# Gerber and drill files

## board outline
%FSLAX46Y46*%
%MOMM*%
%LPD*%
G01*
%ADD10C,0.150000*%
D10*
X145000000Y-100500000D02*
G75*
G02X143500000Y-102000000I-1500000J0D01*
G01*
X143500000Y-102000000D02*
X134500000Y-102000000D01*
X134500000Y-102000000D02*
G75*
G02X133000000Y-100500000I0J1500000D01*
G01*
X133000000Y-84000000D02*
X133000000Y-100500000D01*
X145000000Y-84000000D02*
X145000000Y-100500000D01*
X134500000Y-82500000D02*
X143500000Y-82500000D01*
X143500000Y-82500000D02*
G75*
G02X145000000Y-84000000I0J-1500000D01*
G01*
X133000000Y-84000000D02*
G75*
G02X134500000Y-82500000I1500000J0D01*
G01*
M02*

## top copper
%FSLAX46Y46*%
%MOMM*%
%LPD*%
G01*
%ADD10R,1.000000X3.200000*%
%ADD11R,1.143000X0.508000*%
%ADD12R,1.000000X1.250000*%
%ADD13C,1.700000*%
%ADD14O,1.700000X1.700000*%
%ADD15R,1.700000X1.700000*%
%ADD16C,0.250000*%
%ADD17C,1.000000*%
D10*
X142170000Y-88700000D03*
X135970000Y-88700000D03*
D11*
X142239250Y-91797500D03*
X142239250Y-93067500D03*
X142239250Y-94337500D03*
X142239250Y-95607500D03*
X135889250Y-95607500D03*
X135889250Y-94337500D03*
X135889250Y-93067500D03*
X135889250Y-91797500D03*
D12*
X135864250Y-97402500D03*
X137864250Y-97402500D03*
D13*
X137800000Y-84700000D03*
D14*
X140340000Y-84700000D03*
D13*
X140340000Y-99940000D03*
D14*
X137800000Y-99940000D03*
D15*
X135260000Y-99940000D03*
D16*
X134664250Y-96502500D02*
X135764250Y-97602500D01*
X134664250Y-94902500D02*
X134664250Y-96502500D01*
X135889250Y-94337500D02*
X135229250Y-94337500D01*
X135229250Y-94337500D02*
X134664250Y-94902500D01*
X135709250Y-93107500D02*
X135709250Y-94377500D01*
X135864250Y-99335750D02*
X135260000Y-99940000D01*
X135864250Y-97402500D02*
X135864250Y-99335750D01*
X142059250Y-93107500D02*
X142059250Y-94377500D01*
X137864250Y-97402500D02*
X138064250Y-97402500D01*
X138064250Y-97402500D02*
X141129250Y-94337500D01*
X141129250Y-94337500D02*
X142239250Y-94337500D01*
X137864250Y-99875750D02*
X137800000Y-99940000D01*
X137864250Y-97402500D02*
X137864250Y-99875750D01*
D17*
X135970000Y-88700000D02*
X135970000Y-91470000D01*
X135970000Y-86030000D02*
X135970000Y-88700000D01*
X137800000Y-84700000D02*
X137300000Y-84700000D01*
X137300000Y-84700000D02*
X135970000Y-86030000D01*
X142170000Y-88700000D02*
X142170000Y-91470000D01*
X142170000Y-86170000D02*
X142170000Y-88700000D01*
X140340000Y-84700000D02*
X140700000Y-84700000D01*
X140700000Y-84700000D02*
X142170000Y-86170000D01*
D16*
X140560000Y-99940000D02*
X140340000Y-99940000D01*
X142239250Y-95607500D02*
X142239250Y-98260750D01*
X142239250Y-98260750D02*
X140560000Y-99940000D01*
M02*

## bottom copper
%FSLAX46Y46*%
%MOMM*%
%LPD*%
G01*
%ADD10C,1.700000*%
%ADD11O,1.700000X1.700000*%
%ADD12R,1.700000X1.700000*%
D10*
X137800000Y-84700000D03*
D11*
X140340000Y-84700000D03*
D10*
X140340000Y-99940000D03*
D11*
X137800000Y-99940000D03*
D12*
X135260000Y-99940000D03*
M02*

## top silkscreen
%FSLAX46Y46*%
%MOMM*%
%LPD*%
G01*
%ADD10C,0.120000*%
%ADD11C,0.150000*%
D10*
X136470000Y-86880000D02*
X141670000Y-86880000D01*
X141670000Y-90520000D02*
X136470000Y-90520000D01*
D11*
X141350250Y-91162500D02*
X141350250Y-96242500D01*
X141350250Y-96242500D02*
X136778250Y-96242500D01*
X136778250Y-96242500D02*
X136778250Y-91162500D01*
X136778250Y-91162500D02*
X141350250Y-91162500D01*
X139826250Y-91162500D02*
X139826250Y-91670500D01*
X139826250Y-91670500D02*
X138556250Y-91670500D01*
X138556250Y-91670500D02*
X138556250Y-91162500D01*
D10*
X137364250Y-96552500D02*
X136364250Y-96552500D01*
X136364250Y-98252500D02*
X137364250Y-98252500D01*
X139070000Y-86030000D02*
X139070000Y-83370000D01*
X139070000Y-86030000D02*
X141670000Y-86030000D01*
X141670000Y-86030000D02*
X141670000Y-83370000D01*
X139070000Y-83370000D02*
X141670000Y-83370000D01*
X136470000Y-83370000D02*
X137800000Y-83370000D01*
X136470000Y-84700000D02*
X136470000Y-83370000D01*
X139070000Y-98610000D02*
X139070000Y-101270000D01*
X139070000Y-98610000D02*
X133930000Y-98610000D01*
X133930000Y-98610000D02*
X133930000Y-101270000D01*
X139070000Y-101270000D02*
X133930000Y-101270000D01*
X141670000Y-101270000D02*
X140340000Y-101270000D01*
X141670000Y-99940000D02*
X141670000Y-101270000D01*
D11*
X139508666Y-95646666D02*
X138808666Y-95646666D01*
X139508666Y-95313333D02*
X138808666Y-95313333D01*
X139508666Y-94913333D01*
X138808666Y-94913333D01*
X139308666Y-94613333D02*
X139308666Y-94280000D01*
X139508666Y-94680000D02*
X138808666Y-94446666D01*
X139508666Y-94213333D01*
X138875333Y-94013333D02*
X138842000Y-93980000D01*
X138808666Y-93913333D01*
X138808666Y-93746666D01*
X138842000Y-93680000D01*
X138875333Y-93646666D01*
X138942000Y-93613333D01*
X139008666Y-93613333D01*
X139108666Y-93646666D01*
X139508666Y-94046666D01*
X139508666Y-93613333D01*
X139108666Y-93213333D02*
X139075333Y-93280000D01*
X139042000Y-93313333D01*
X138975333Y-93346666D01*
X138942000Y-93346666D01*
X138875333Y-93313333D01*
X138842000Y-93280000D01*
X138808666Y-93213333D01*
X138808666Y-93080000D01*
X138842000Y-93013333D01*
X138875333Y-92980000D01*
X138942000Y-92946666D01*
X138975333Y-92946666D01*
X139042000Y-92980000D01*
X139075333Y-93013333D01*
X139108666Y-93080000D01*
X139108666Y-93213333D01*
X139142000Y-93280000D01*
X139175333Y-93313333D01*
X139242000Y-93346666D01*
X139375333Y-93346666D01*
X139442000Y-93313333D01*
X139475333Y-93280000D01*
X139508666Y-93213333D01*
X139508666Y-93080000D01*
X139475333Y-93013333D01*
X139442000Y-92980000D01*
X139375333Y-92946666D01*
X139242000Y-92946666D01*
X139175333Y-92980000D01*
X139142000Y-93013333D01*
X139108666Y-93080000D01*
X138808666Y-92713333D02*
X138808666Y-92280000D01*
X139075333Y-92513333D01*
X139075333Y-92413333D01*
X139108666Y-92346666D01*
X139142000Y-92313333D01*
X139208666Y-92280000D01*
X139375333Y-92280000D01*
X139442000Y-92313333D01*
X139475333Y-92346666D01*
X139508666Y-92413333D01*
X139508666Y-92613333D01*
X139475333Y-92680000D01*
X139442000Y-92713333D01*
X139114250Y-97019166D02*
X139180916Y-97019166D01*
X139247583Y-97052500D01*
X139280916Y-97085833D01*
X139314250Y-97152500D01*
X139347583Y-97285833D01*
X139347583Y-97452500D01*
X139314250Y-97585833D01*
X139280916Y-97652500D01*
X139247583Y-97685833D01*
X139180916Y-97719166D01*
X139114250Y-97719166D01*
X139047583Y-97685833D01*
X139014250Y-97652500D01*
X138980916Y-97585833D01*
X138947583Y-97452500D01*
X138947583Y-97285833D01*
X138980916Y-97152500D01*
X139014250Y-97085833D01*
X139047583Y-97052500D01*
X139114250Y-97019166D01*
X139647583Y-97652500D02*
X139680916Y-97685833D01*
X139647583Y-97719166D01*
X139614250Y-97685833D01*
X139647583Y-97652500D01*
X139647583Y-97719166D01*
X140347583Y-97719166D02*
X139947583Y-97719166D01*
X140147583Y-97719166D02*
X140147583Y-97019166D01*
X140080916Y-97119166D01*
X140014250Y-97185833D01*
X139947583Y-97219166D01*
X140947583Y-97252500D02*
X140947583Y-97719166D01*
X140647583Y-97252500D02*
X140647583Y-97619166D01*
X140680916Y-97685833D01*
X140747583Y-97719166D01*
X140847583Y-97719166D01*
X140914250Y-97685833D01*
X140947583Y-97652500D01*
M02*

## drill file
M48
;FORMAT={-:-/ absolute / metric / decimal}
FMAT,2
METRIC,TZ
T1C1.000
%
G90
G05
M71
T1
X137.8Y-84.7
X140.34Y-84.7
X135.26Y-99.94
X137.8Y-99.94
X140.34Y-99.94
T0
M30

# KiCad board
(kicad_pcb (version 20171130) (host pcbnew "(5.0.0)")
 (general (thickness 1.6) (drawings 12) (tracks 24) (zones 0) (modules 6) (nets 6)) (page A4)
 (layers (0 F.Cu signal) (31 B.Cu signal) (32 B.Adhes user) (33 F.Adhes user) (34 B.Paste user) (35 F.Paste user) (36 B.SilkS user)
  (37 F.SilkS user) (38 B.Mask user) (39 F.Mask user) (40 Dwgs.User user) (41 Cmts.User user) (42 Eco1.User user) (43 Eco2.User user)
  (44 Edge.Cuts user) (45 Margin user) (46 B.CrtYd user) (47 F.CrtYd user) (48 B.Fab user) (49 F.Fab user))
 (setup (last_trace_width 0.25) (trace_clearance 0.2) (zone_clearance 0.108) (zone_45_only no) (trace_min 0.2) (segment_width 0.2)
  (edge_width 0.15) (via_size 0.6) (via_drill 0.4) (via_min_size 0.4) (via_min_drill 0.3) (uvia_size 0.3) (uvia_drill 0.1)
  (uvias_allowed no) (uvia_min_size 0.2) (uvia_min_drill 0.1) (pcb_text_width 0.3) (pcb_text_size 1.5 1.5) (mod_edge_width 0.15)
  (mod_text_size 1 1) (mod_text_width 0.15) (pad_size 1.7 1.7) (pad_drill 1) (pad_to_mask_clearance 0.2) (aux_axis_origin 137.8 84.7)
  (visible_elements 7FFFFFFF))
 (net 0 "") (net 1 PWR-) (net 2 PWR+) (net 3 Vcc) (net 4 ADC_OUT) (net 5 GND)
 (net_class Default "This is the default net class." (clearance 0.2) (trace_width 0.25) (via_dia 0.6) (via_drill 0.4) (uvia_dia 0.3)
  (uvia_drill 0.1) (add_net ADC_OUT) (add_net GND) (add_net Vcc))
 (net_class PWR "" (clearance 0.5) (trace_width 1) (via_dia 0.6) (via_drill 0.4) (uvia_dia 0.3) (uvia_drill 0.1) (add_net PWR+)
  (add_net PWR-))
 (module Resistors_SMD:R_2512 (layer F.Cu) (at 139.07 88.7 180)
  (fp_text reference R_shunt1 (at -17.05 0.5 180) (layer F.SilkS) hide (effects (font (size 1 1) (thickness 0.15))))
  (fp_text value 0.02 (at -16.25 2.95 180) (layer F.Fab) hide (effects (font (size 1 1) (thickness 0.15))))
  (fp_line (start 2.6 1.82) (end -2.6 1.82) (layer F.SilkS) (width 0.12))
  (fp_line (start -2.6 -1.82) (end 2.6 -1.82) (layer F.SilkS) (width 0.12))
  (pad 1 smd rect (at -3.1 0 180) (size 1 3.2) (layers F.Cu F.Paste F.Mask) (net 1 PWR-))
  (pad 2 smd rect (at 3.1 0 180) (size 1 3.2) (layers F.Cu F.Paste F.Mask) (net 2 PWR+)))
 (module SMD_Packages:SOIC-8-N (layer F.Cu) (at 139.06425 93.7025 270)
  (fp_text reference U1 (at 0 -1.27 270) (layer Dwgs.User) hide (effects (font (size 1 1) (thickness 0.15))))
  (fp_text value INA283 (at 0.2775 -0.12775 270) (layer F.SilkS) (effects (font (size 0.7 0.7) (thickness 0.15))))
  (fp_line (start -2.54 -2.286) (end 2.54 -2.286) (layer F.SilkS) (width 0.15))
  (fp_line (start 2.54 -2.286) (end 2.54 2.286) (layer F.SilkS) (width 0.15))
  (fp_line (start 2.54 2.286) (end -2.54 2.286) (layer F.SilkS) (width 0.15))
  (fp_line (start -2.54 2.286) (end -2.54 -2.286) (layer F.SilkS) (width 0.15))
  (fp_line (start -2.54 -0.762) (end -2.032 -0.762) (layer F.SilkS) (width 0.15))
  (fp_line (start -2.032 -0.762) (end -2.032 0.508) (layer F.SilkS) (width 0.15))
  (fp_line (start -2.032 0.508) (end -2.54 0.508) (layer F.SilkS) (width 0.15))
  (pad 8 smd rect (at -1.905 -3.175 270) (size 0.508 1.143) (layers F.Cu F.Paste F.Mask) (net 1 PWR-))
  (pad 7 smd rect (at -0.635 -3.175 270) (size 0.508 1.143) (layers F.Cu F.Paste F.Mask) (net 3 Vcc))
  (pad 6 smd rect (at 0.635 -3.175 270) (size 0.508 1.143) (layers F.Cu F.Paste F.Mask) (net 3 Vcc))
  (pad 5 smd rect (at 1.905 -3.175 270) (size 0.508 1.143) (layers F.Cu F.Paste F.Mask) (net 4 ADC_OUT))
  (pad 4 smd rect (at 1.905 3.175 270) (size 0.508 1.143) (layers F.Cu F.Paste F.Mask))
  (pad 3 smd rect (at 0.635 3.175 270) (size 0.508 1.143) (layers F.Cu F.Paste F.Mask) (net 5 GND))
  (pad 2 smd rect (at -0.635 3.175 270) (size 0.508 1.143) (layers F.Cu F.Paste F.Mask) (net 5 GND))
  (pad 1 smd rect (at -1.905 3.175 270) (size 0.508 1.143) (layers F.Cu F.Paste F.Mask) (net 2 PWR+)))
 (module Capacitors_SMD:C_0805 (layer F.Cu) (at 136.86425 97.4025)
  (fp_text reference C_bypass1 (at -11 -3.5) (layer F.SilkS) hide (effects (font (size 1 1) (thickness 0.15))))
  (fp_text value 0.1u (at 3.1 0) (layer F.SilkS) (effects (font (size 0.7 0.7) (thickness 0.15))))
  (fp_line (start 0.5 -0.85) (end -0.5 -0.85) (layer F.SilkS) (width 0.12))
  (fp_line (start -0.5 0.85) (end 0.5 0.85) (layer F.SilkS) (width 0.12))
  (pad 1 smd rect (at -1 0) (size 1 1.25) (layers F.Cu F.Paste F.Mask) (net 5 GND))
  (pad 2 smd rect (at 1 0) (size 1 1.25) (layers F.Cu F.Paste F.Mask) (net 3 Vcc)))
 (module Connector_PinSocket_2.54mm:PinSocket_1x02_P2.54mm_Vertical (layer F.Cu) (at 137.8 84.7 90)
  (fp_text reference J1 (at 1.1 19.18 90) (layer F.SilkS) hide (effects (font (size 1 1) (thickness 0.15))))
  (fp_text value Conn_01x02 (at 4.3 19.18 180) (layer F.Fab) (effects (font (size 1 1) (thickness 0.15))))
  (fp_line (start -1.33 1.27) (end 1.33 1.27) (layer F.SilkS) (width 0.12))
  (fp_line (start -1.33 1.27) (end -1.33 3.87) (layer F.SilkS) (width 0.12))
  (fp_line (start -1.33 3.87) (end 1.33 3.87) (layer F.SilkS) (width 0.12))
  (fp_line (start 1.33 1.27) (end 1.33 3.87) (layer F.SilkS) (width 0.12))
  (fp_line (start 1.33 -1.33) (end 1.33 0) (layer F.SilkS) (width 0.12))
  (fp_line (start 0 -1.33) (end 1.33 -1.33) (layer F.SilkS) (width 0.12))
  (pad 1 thru_hole circle (at 0 0 90) (size 1.7 1.7) (drill 1) (layers *.Cu *.Mask) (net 2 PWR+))
  (pad 2 thru_hole oval (at 0 2.54 90) (size 1.7 1.7) (drill 1) (layers *.Cu *.Mask) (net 1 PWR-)))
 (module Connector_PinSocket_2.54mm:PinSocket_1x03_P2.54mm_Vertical (layer F.Cu) (at 140.34 99.94 270)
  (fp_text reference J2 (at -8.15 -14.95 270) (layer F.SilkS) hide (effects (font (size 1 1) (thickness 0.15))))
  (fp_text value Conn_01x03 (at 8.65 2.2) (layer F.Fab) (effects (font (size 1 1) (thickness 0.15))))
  (fp_line (start -1.33 1.27) (end 1.33 1.27) (layer F.SilkS) (width 0.12))
  (fp_line (start -1.33 1.27) (end -1.33 6.41) (layer F.SilkS) (width 0.12))
  (fp_line (start -1.33 6.41) (end 1.33 6.41) (layer F.SilkS) (width 0.12))
  (fp_line (start 1.33 1.27) (end 1.33 6.41) (layer F.SilkS) (width 0.12))
  (fp_line (start 1.33 -1.33) (end 1.33 0) (layer F.SilkS) (width 0.12))
  (fp_line (start 0 -1.33) (end 1.33 -1.33) (layer F.SilkS) (width 0.12))
  (pad 1 thru_hole circle (at 0 0 270) (size 1.7 1.7) (drill 1) (layers *.Cu *.Mask) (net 4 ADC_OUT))
  (pad 2 thru_hole oval (at 0 2.54 270) (size 1.7 1.7) (drill 1) (layers *.Cu *.Mask) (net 3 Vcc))
  (pad 3 thru_hole rect (at 0 5.08 270) (size 1.7 1.7) (drill 1) (layers *.Cu *.Mask) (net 5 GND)))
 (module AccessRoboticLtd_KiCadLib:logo (layer B.Cu) (at 139 90.5 180)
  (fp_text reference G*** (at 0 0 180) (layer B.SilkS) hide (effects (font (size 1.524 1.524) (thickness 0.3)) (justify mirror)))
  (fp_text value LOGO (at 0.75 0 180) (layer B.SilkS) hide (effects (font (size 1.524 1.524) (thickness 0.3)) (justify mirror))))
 (gr_arc (start 143.5 100.5) (end 143.5 102) (angle -90) (layer Edge.Cuts) (width 0.15))
 (gr_line (start 143.5 102) (end 134.5 102) (layer Edge.Cuts) (width 0.15))
 (gr_arc (start 134.5 100.5) (end 133 100.5) (angle -90) (layer Edge.Cuts) (width 0.15))
 (gr_line (start 133 84) (end 133 100.5) (layer Edge.Cuts) (width 0.15))
 (gr_line (start 145 84) (end 145 100.5) (layer Edge.Cuts) (width 0.15))
 (gr_line (start 134.5 82.5) (end 143.5 82.5) (layer Edge.Cuts) (width 0.15))
 (gr_arc (start 143.5 84) (end 145 84) (angle -90) (layer Edge.Cuts) (width 0.15))
 (gr_arc (start 134.5 84) (end 134.5 82.5) (angle -90) (layer Edge.Cuts) (width 0.15))
 (segment (start 134.66425 96.5025) (end 135.76425 97.6025) (width 0.25) (layer F.Cu) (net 5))
 (segment (start 134.66425 94.9025) (end 134.66425 96.5025) (width 0.25) (layer F.Cu) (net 5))
 (segment (start 135.88925 94.3375) (end 135.22925 94.3375) (width 0.25) (layer F.Cu) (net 5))
 (segment (start 135.22925 94.3375) (end 134.66425 94.9025) (width 0.25) (layer F.Cu) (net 5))
 (segment (start 135.70925 93.1075) (end 135.70925 94.3775) (width 0.25) (layer F.Cu) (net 5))
 (segment (start 135.86425 99.33575) (end 135.26 99.94) (width 0.25) (layer F.Cu) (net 5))
 (segment (start 135.86425 97.4025) (end 135.86425 99.33575) (width 0.25) (layer F.Cu) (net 5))
 (segment (start 142.05925 93.1075) (end 142.05925 94.3775) (width 0.25) (layer F.Cu) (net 3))
 (segment (start 137.86425 97.4025) (end 138.06425 97.4025) (width 0.25) (layer F.Cu) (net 3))
 (segment (start 138.06425 97.4025) (end 141.12925 94.3375) (width 0.25) (layer F.Cu) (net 3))
 (segment (start 141.12925 94.3375) (end 142.23925 94.3375) (width 0.25) (layer F.Cu) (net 3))
 (segment (start 137.86425 99.87575) (end 137.8 99.94) (width 0.25) (layer F.Cu) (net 3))
 (segment (start 137.86425 97.4025) (end 137.86425 99.87575) (width 0.25) (layer F.Cu) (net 3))
 (segment (start 135.97 88.7) (end 135.97 91.47) (width 1) (layer F.Cu) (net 2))
 (segment (start 135.97 86.03) (end 135.97 88.7) (width 1) (layer F.Cu) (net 2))
 (segment (start 137.8 84.7) (end 137.3 84.7) (width 1) (layer F.Cu) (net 2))
 (segment (start 137.3 84.7) (end 135.97 86.03) (width 1) (layer F.Cu) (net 2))
 (segment (start 142.17 88.7) (end 142.17 91.47) (width 1) (layer F.Cu) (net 1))
 (segment (start 142.17 86.17) (end 142.17 88.7) (width 1) (layer F.Cu) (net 1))
 (segment (start 140.34 84.7) (end 140.7 84.7) (width 1) (layer F.Cu) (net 1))
 (segment (start 140.7 84.7) (end 142.17 86.17) (width 1) (layer F.Cu) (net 1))
 (segment (start 140.56 99.94) (end 140.34 99.94) (width 0.25) (layer F.Cu) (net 4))
 (segment (start 142.23925 95.6075) (end 142.23925 98.26075) (width 0.25) (layer F.Cu) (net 4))
 (segment (start 142.23925 98.26075) (end 140.56 99.94) (width 0.25) (layer F.Cu) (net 4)))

